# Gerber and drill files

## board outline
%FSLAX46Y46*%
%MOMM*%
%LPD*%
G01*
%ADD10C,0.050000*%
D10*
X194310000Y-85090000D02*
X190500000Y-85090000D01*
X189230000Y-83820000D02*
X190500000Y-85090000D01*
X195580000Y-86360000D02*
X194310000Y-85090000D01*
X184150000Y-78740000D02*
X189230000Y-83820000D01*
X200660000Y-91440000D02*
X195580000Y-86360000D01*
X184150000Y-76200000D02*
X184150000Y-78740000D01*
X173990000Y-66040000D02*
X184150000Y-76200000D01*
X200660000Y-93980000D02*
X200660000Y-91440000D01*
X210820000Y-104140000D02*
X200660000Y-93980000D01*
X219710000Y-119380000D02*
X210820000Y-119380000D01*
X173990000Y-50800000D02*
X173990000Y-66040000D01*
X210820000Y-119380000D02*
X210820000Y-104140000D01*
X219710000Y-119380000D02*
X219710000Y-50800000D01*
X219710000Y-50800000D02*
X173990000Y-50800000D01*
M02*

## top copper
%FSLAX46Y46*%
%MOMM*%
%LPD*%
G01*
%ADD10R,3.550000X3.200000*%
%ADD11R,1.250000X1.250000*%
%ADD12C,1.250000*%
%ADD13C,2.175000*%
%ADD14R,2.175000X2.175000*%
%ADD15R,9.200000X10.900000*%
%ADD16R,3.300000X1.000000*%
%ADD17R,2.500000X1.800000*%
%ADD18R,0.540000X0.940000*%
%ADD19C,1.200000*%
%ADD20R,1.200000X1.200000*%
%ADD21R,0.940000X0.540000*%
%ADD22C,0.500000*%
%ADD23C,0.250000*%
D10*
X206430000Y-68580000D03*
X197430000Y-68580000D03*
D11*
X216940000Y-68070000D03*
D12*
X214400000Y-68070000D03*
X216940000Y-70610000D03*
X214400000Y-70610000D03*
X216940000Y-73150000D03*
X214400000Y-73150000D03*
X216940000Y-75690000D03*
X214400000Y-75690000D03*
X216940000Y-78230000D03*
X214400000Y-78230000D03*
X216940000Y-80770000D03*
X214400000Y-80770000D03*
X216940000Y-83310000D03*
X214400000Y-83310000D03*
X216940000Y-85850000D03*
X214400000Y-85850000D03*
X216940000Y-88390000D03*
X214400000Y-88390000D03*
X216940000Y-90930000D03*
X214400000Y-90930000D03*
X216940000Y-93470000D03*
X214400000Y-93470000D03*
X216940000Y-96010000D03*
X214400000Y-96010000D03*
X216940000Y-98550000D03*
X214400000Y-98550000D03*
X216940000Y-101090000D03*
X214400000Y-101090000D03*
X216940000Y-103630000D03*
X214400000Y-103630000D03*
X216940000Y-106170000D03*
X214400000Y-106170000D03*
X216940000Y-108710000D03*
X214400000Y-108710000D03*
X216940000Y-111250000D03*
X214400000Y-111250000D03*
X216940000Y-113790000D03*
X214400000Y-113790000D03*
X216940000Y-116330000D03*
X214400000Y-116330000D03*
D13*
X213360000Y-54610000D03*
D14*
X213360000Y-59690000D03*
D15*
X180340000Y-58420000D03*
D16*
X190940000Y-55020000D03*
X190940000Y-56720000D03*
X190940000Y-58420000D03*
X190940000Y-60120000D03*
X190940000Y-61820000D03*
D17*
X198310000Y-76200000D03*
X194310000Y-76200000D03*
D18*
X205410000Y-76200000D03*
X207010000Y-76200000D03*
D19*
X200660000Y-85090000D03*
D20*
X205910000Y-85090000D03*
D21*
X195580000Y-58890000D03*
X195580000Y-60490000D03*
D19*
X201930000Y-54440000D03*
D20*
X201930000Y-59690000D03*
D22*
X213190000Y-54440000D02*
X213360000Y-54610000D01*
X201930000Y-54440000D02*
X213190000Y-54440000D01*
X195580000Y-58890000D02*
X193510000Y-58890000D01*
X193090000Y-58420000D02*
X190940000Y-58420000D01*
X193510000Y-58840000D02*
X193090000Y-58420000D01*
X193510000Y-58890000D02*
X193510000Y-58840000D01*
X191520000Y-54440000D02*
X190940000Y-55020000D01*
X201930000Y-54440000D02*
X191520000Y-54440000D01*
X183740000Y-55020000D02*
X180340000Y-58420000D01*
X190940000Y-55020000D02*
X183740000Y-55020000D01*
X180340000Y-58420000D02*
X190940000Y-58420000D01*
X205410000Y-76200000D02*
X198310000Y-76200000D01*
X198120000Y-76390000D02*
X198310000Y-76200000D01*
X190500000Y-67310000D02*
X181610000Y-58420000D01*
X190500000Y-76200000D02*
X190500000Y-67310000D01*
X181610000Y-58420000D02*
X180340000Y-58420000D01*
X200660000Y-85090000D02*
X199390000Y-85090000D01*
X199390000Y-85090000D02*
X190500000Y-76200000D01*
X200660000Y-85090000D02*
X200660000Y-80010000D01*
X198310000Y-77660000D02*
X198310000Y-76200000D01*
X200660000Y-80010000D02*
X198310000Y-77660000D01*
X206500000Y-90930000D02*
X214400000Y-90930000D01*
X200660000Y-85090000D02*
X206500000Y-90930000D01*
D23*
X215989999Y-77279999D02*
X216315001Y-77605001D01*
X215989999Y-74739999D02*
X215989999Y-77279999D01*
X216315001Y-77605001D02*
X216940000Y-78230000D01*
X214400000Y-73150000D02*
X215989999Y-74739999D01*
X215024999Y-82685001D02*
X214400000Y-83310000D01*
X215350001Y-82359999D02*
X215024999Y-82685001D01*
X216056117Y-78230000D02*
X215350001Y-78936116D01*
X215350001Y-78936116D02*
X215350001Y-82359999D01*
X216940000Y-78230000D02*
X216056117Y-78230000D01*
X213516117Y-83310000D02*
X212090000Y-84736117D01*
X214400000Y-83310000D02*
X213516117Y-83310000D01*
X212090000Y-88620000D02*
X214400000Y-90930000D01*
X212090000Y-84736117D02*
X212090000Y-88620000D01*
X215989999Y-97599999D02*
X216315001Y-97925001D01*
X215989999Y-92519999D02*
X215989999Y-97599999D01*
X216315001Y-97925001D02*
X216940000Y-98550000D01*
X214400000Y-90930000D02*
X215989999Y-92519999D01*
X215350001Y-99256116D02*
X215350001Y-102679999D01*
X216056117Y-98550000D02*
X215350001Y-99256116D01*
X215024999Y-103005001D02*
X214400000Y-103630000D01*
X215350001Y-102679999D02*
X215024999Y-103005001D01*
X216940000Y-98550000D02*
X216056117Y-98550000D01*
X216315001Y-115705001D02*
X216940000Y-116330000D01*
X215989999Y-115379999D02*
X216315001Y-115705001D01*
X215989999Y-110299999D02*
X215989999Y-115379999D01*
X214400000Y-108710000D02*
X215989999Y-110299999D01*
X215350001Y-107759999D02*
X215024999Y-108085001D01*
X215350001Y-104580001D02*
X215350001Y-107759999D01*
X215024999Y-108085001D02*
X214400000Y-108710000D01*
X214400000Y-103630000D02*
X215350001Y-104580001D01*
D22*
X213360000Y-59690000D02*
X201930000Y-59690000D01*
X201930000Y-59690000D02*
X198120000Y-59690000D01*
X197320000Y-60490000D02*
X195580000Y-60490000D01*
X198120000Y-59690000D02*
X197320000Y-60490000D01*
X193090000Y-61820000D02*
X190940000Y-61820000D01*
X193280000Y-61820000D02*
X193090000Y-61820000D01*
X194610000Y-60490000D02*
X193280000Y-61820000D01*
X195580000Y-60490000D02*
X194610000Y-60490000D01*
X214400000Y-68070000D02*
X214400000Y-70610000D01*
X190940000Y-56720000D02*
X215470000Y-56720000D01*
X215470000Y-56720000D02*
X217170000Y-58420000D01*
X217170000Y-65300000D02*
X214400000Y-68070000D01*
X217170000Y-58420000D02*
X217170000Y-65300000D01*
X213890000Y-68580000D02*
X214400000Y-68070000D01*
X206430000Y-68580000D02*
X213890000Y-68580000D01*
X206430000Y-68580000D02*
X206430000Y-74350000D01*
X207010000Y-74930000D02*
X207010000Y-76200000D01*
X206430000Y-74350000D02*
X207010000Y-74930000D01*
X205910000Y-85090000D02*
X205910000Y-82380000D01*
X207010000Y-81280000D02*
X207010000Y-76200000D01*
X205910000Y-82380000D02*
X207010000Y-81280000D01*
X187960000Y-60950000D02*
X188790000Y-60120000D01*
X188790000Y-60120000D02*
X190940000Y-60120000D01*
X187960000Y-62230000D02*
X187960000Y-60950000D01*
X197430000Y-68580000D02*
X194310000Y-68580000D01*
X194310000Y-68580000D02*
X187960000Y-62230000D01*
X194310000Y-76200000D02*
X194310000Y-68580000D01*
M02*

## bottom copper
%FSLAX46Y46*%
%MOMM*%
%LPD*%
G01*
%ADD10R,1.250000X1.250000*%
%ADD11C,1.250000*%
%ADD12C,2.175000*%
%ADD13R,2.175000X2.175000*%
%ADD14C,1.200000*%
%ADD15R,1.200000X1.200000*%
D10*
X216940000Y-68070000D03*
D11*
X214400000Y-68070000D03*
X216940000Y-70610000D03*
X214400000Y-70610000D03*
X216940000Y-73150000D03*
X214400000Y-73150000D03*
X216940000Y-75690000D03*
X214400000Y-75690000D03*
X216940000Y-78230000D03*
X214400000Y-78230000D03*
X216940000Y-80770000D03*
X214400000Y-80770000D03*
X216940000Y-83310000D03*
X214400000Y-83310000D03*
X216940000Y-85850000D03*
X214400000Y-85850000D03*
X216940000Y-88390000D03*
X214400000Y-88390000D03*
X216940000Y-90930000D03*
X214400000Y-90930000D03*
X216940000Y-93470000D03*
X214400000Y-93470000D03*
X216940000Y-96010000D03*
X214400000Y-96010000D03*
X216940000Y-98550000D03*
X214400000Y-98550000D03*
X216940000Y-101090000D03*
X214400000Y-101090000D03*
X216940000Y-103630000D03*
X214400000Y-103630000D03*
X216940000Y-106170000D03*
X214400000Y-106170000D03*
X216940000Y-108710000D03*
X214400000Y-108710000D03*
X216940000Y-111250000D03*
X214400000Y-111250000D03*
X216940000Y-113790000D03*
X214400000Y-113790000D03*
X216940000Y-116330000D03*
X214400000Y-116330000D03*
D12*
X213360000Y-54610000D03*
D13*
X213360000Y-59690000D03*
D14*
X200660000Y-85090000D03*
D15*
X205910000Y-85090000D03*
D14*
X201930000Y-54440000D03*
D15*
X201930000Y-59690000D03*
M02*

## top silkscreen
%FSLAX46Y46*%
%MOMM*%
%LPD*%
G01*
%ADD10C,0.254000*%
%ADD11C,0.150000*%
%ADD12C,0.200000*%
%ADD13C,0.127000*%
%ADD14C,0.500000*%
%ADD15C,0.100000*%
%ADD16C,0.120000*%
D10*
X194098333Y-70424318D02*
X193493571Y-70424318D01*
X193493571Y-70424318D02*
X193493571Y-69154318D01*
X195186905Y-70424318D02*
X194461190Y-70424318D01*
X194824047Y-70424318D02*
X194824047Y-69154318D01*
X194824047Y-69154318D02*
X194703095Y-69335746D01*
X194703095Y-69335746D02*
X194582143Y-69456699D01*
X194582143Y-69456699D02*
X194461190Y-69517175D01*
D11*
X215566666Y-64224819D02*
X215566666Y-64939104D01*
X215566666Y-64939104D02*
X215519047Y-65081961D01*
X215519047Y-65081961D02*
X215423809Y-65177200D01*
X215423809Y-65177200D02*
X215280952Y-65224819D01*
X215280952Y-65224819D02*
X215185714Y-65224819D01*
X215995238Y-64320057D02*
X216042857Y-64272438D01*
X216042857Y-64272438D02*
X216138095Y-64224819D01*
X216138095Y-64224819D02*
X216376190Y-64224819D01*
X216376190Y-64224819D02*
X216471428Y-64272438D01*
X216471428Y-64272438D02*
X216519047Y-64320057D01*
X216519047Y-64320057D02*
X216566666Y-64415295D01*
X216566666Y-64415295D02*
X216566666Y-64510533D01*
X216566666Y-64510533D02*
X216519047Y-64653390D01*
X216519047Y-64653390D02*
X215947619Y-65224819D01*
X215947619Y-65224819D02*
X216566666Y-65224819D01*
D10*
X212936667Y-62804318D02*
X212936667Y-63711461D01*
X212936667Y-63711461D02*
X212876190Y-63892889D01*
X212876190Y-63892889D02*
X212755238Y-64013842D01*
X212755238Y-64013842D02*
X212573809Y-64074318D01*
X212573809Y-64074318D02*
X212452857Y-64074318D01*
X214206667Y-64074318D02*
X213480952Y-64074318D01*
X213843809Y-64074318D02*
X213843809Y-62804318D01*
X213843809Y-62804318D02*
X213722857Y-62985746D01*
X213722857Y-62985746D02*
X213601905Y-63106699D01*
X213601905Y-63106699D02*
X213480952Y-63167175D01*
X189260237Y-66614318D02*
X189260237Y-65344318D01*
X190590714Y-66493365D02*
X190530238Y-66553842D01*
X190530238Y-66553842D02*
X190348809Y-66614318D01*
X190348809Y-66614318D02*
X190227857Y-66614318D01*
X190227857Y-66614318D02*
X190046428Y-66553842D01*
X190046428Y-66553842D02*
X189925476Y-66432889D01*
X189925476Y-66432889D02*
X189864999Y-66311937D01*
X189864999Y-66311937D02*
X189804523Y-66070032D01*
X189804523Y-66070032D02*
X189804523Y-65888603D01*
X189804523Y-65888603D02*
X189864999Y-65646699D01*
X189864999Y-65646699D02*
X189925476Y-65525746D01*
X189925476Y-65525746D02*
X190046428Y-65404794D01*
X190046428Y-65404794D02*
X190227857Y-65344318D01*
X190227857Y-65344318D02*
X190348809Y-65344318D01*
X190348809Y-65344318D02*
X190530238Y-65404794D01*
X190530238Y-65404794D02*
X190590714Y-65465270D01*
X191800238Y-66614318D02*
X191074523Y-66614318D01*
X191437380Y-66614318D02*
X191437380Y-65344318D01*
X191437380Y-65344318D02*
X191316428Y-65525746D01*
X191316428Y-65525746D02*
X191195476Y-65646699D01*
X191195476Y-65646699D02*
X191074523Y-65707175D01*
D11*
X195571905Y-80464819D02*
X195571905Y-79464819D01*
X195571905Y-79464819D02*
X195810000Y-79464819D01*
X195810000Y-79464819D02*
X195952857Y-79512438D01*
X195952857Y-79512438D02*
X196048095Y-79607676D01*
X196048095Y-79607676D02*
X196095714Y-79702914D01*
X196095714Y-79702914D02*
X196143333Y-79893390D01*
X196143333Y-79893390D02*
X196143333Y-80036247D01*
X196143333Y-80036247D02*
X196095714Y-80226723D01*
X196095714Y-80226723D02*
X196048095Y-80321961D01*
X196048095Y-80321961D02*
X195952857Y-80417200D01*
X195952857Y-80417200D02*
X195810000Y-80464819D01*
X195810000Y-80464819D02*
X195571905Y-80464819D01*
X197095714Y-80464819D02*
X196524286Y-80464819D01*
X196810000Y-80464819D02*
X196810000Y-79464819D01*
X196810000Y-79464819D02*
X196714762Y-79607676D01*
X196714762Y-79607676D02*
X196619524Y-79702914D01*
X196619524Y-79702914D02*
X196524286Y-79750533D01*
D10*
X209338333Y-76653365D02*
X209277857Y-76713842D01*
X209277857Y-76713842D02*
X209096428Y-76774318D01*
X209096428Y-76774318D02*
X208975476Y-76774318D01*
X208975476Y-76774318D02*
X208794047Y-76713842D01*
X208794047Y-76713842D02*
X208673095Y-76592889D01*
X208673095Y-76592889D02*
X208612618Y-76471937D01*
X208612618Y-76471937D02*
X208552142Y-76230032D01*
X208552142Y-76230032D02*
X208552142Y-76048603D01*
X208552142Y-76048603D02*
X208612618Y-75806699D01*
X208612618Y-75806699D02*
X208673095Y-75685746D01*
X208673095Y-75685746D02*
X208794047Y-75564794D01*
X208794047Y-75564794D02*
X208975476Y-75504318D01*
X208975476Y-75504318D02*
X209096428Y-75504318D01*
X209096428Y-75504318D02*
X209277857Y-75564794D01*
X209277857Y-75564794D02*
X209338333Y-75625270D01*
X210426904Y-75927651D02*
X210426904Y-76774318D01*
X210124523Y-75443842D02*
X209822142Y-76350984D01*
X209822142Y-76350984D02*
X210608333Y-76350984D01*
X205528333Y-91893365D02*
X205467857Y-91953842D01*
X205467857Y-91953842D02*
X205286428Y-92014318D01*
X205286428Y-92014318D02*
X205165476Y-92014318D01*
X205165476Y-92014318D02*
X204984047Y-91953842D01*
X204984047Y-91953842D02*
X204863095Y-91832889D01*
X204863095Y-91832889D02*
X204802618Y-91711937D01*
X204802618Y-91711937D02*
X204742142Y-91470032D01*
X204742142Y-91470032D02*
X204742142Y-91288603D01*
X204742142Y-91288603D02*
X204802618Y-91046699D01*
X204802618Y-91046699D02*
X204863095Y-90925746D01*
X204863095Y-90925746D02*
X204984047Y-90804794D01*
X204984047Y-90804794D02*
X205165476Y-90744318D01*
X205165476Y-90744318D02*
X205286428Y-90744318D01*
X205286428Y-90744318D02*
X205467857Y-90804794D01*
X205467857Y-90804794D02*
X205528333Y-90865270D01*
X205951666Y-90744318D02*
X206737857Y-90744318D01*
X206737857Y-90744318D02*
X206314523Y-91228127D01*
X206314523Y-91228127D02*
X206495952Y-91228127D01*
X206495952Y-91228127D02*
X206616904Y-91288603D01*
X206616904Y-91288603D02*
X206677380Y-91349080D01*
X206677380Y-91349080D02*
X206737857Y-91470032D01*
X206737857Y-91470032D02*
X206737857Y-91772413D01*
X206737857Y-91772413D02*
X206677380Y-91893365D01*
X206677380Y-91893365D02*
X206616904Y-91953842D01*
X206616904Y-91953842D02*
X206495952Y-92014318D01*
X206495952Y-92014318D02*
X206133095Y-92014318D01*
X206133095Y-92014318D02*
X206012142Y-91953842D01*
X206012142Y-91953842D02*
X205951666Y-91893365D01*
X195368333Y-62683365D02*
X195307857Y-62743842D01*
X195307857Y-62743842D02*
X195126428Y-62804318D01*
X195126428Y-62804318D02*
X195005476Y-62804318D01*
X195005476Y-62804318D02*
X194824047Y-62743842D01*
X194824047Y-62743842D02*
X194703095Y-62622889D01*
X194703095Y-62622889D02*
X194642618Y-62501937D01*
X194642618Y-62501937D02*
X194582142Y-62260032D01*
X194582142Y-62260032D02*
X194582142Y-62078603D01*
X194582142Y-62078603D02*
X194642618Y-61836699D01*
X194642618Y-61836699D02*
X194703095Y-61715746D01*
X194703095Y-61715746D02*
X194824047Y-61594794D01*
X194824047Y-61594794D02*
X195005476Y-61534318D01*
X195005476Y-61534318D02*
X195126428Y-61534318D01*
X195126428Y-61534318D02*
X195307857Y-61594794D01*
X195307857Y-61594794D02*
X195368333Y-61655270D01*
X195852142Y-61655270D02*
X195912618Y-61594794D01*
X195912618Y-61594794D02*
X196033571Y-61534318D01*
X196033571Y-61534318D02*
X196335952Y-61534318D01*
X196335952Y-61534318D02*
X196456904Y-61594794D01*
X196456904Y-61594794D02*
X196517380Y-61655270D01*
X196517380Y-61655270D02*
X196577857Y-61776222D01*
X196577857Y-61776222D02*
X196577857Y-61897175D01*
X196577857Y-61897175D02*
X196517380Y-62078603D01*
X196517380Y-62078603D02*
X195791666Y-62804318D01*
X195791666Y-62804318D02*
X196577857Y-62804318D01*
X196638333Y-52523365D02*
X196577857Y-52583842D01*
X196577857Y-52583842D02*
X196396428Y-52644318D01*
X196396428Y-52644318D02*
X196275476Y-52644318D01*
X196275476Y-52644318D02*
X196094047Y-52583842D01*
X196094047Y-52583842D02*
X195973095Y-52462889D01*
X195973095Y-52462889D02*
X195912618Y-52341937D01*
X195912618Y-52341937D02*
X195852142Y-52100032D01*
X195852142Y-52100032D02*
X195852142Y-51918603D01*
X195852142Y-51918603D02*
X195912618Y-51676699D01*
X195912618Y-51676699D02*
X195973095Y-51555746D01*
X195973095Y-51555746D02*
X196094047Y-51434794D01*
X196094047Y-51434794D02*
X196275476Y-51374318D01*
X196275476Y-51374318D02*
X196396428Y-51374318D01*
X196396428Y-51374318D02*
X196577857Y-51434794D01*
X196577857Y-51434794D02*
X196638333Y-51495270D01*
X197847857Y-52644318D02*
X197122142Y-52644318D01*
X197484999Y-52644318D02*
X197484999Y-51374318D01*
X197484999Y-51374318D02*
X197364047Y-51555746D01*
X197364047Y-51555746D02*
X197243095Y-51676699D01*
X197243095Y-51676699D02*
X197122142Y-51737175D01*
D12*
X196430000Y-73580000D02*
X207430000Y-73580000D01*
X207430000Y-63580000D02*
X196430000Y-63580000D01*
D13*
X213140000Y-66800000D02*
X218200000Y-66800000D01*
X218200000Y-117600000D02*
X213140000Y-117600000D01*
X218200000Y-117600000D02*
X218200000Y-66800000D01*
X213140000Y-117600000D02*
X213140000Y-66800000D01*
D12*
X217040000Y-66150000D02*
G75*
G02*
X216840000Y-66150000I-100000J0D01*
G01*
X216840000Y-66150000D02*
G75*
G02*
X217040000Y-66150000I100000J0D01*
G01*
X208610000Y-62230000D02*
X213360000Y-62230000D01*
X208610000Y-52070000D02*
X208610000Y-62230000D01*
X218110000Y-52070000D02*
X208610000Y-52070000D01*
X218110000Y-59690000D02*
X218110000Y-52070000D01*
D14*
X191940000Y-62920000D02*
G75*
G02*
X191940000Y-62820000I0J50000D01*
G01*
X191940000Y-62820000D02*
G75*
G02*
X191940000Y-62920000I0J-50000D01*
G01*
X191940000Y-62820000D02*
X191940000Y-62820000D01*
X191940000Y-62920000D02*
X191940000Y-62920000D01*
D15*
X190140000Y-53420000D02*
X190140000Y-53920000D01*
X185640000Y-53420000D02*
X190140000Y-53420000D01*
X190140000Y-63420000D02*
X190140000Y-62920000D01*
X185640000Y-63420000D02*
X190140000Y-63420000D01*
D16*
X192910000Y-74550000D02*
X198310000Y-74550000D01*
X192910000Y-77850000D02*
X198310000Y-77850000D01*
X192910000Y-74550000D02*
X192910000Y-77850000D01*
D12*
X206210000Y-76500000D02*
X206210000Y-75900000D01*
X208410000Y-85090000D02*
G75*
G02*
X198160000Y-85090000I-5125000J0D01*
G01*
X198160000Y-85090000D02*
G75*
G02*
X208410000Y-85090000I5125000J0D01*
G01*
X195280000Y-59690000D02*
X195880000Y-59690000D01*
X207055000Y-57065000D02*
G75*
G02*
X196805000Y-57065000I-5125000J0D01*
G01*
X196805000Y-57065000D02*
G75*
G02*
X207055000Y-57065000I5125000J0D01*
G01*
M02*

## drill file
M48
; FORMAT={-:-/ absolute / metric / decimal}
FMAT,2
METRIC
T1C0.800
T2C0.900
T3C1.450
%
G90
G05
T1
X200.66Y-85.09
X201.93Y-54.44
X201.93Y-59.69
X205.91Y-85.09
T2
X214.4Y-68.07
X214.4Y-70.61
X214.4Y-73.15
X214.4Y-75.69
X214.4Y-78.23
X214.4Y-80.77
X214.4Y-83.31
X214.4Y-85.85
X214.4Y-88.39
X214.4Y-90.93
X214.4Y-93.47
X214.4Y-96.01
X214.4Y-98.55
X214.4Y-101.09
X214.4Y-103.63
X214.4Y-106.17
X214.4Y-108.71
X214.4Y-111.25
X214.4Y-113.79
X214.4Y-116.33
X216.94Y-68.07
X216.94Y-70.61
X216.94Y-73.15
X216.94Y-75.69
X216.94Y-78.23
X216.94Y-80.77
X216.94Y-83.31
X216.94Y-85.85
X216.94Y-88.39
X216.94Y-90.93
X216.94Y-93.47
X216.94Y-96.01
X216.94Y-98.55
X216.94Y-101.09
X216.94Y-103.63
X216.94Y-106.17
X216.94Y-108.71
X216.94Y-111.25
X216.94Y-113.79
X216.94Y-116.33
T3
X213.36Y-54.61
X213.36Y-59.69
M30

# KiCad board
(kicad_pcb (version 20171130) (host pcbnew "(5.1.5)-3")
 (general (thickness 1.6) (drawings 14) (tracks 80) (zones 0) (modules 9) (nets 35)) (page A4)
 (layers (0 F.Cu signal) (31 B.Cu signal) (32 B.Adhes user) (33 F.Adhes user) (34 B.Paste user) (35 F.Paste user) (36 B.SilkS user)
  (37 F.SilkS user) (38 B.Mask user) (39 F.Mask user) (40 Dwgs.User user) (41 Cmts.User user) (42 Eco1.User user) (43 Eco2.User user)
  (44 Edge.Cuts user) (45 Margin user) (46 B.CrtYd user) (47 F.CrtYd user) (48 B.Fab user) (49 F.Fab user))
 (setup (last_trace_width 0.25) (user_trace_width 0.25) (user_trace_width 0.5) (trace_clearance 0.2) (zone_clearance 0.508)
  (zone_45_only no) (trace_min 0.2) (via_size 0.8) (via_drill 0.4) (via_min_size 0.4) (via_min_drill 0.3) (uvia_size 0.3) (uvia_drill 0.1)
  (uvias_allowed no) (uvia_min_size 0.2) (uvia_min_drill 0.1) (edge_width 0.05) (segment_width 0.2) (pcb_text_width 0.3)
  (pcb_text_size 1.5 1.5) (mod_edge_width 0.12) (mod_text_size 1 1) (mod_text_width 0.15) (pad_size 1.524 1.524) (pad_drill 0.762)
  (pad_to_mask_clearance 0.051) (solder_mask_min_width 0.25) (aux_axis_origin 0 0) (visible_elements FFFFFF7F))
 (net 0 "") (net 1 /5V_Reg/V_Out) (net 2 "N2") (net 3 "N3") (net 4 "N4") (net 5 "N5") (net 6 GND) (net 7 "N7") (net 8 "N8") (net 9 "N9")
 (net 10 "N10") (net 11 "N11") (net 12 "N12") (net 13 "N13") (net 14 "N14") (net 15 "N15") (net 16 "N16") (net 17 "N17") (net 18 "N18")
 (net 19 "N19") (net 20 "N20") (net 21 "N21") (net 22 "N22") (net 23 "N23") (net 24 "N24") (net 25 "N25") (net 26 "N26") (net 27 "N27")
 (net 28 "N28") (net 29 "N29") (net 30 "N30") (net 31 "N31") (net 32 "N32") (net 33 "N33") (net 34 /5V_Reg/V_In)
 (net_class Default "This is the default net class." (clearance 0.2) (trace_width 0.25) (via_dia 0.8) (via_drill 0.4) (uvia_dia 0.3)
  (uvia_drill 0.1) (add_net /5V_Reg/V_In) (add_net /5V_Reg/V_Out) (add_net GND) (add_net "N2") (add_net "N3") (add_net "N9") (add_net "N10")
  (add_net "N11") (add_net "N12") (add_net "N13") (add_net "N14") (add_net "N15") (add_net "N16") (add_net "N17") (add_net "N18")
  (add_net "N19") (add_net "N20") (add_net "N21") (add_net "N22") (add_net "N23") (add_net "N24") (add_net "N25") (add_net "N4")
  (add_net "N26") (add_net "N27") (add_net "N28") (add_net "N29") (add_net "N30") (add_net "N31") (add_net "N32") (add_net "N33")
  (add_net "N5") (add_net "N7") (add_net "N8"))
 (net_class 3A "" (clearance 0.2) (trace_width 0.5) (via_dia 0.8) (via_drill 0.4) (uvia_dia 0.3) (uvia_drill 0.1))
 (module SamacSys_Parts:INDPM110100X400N (layer F.Cu) (at 201.93 68.58)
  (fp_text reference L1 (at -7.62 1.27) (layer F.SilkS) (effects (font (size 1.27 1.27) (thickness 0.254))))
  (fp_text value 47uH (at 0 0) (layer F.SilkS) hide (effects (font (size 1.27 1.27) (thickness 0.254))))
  (fp_line (start -5.5 5) (end 5.5 5) (layer F.SilkS) (width 0.2))
  (fp_line (start 5.5 -5) (end -5.5 -5) (layer F.SilkS) (width 0.2))
  (pad 2 smd rect (at 4.5 0 90) (size 3.2 3.55) (layers F.Cu F.Paste F.Mask) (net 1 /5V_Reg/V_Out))
  (pad 1 smd rect (at -4.5 0 90) (size 3.2 3.55) (layers F.Cu F.Paste F.Mask) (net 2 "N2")))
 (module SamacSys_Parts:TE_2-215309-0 (layer F.Cu) (at 216.94 68.07 270)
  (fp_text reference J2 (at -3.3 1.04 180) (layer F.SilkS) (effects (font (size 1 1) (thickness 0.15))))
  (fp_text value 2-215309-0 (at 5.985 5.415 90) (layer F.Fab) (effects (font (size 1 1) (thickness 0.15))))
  (fp_line (start -1.27 3.8) (end -1.27 -1.26) (layer F.SilkS) (width 0.127))
  (fp_line (start 49.53 -1.26) (end 49.53 3.8) (layer F.SilkS) (width 0.127))
  (fp_line (start 49.53 -1.26) (end -1.27 -1.26) (layer F.SilkS) (width 0.127))
  (fp_line (start 49.53 3.8) (end -1.27 3.8) (layer F.SilkS) (width 0.127))
  (fp_circle (center -1.92 0) (end -1.82 0) (layer F.SilkS) (width 0.2))
  (pad 1 thru_hole rect (at 0 0 270) (size 1.25 1.25) (drill 0.9) (layers *.Cu *.Mask) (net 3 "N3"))
  (pad 2 thru_hole circle (at 0 2.54 270) (size 1.25 1.25) (drill 0.9) (layers *.Cu *.Mask) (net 1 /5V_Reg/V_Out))
  (pad 3 thru_hole circle (at 2.54 0 270) (size 1.25 1.25) (drill 0.9) (layers *.Cu *.Mask) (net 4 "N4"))
  (pad 4 thru_hole circle (at 2.54 2.54 270) (size 1.25 1.25) (drill 0.9) (layers *.Cu *.Mask) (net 1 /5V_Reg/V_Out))
  (pad 5 thru_hole circle (at 5.08 0 270) (size 1.25 1.25) (drill 0.9) (layers *.Cu *.Mask) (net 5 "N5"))
  (pad 6 thru_hole circle (at 5.08 2.54 270) (size 1.25 1.25) (drill 0.9) (layers *.Cu *.Mask) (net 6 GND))
  (pad 7 thru_hole circle (at 7.62 0 270) (size 1.25 1.25) (drill 0.9) (layers *.Cu *.Mask) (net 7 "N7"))
  (pad 8 thru_hole circle (at 7.62 2.54 270) (size 1.25 1.25) (drill 0.9) (layers *.Cu *.Mask) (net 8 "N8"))
  (pad 9 thru_hole circle (at 10.16 0 270) (size 1.25 1.25) (drill 0.9) (layers *.Cu *.Mask) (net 6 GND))
  (pad 10 thru_hole circle (at 10.16 2.54 270) (size 1.25 1.25) (drill 0.9) (layers *.Cu *.Mask) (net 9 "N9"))
  (pad 11 thru_hole circle (at 12.7 0 270) (size 1.25 1.25) (drill 0.9) (layers *.Cu *.Mask) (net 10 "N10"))
  (pad 12 thru_hole circle (at 12.7 2.54 270) (size 1.25 1.25) (drill 0.9) (layers *.Cu *.Mask) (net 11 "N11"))
  (pad 13 thru_hole circle (at 15.24 0 270) (size 1.25 1.25) (drill 0.9) (layers *.Cu *.Mask) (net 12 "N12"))
  (pad 14 thru_hole circle (at 15.24 2.54 270) (size 1.25 1.25) (drill 0.9) (layers *.Cu *.Mask) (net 6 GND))
  (pad 15 thru_hole circle (at 17.78 0 270) (size 1.25 1.25) (drill 0.9) (layers *.Cu *.Mask) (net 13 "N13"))
  (pad 16 thru_hole circle (at 17.78 2.54 270) (size 1.25 1.25) (drill 0.9) (layers *.Cu *.Mask) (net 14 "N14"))
  (pad 17 thru_hole circle (at 20.32 0 270) (size 1.25 1.25) (drill 0.9) (layers *.Cu *.Mask) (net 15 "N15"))
  (pad 18 thru_hole circle (at 20.32 2.54 270) (size 1.25 1.25) (drill 0.9) (layers *.Cu *.Mask) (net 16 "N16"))
  (pad 19 thru_hole circle (at 22.86 0 270) (size 1.25 1.25) (drill 0.9) (layers *.Cu *.Mask) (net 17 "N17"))
  (pad 20 thru_hole circle (at 22.86 2.54 270) (size 1.25 1.25) (drill 0.9) (layers *.Cu *.Mask) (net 6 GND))
  (pad 21 thru_hole circle (at 25.4 0 270) (size 1.25 1.25) (drill 0.9) (layers *.Cu *.Mask) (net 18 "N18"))
  (pad 22 thru_hole circle (at 25.4 2.54 270) (size 1.25 1.25) (drill 0.9) (layers *.Cu *.Mask) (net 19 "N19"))
  (pad 23 thru_hole circle (at 27.94 0 270) (size 1.25 1.25) (drill 0.9) (layers *.Cu *.Mask) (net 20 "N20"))
  (pad 24 thru_hole circle (at 27.94 2.54 270) (size 1.25 1.25) (drill 0.9) (layers *.Cu *.Mask) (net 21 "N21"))
  (pad 25 thru_hole circle (at 30.48 0 270) (size 1.25 1.25) (drill 0.9) (layers *.Cu *.Mask) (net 6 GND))
  (pad 26 thru_hole circle (at 30.48 2.54 270) (size 1.25 1.25) (drill 0.9) (layers *.Cu *.Mask) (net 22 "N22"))
  (pad 27 thru_hole circle (at 33.02 0 270) (size 1.25 1.25) (drill 0.9) (layers *.Cu *.Mask) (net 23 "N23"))
  (pad 28 thru_hole circle (at 33.02 2.54 270) (size 1.25 1.25) (drill 0.9) (layers *.Cu *.Mask) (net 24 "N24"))
  (pad 29 thru_hole circle (at 35.56 0 270) (size 1.25 1.25) (drill 0.9) (layers *.Cu *.Mask) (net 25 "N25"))
  (pad 30 thru_hole circle (at 35.56 2.54 270) (size 1.25 1.25) (drill 0.9) (layers *.Cu *.Mask) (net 6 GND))
  (pad 31 thru_hole circle (at 38.1 0 270) (size 1.25 1.25) (drill 0.9) (layers *.Cu *.Mask) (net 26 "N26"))
  (pad 32 thru_hole circle (at 38.1 2.54 270) (size 1.25 1.25) (drill 0.9) (layers *.Cu *.Mask) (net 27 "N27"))
  (pad 33 thru_hole circle (at 40.64 0 270) (size 1.25 1.25) (drill 0.9) (layers *.Cu *.Mask) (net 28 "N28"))
  (pad 34 thru_hole circle (at 40.64 2.54 270) (size 1.25 1.25) (drill 0.9) (layers *.Cu *.Mask) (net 6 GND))
  (pad 35 thru_hole circle (at 43.18 0 270) (size 1.25 1.25) (drill 0.9) (layers *.Cu *.Mask) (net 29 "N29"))
  (pad 36 thru_hole circle (at 43.18 2.54 270) (size 1.25 1.25) (drill 0.9) (layers *.Cu *.Mask) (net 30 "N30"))
  (pad 37 thru_hole circle (at 45.72 0 270) (size 1.25 1.25) (drill 0.9) (layers *.Cu *.Mask) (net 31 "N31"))
  (pad 38 thru_hole circle (at 45.72 2.54 270) (size 1.25 1.25) (drill 0.9) (layers *.Cu *.Mask) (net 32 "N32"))
  (pad 39 thru_hole circle (at 48.26 0 270) (size 1.25 1.25) (drill 0.9) (layers *.Cu *.Mask) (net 6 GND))
  (pad 40 thru_hole circle (at 48.26 2.54 270) (size 1.25 1.25) (drill 0.9) (layers *.Cu *.Mask) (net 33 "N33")))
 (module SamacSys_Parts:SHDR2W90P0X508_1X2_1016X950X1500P (layer F.Cu) (at 213.36 59.69 90)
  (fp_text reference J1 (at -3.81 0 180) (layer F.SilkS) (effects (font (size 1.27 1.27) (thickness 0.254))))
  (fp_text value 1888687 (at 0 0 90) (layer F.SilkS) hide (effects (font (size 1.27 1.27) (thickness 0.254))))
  (fp_line (start -2.54 -4.75) (end -2.54 0) (layer F.SilkS) (width 0.2))
  (fp_line (start 7.62 -4.75) (end -2.54 -4.75) (layer F.SilkS) (width 0.2))
  (fp_line (start 7.62 4.75) (end 7.62 -4.75) (layer F.SilkS) (width 0.2))
  (fp_line (start 0 4.75) (end 7.62 4.75) (layer F.SilkS) (width 0.2))
  (pad 2 thru_hole circle (at 5.08 0 90) (size 2.175 2.175) (drill 1.45) (layers *.Cu *.Mask) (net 6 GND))
  (pad 1 thru_hole rect (at 0 0 90) (size 2.175 2.175) (drill 1.45) (layers *.Cu *.Mask) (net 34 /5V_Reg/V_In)))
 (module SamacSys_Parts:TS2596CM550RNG (layer F.Cu) (at 185.64 58.42 90)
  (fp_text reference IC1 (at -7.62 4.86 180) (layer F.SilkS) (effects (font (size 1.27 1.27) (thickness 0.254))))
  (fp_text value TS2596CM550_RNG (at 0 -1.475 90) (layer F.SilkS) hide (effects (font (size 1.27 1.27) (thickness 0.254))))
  (fp_arc (start -4.45 6.3) (end -4.4 6.3) (angle -180) (layer F.SilkS) (width 0.5))
  (fp_arc (start -4.45 6.3) (end -4.5 6.3) (angle -180) (layer F.SilkS) (width 0.5))
  (fp_line (start -4.4 6.3) (end -4.4 6.3) (layer F.SilkS) (width 0.5))
  (fp_line (start -4.5 6.3) (end -4.5 6.3) (layer F.SilkS) (width 0.5))
  (fp_line (start 5 4.5) (end 4.5 4.5) (layer F.SilkS) (width 0.1))
  (fp_line (start 5 0) (end 5 4.5) (layer F.SilkS) (width 0.1))
  (fp_line (start -5 4.5) (end -4.5 4.5) (layer F.SilkS) (width 0.1))
  (fp_line (start -5 0) (end -5 4.5) (layer F.SilkS) (width 0.1))
  (pad 6 smd rect (at 0 -5.3 180) (size 9.2 10.9) (layers F.Cu F.Paste F.Mask) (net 6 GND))
  (pad 5 smd rect (at 3.4 5.3 90) (size 1 3.3) (layers F.Cu F.Paste F.Mask) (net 6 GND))
  (pad 4 smd rect (at 1.7 5.3 90) (size 1 3.3) (layers F.Cu F.Paste F.Mask) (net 1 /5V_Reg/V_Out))
  (pad 3 smd rect (at 0 5.3 90) (size 1 3.3) (layers F.Cu F.Paste F.Mask) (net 6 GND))
  (pad 2 smd rect (at -1.7 5.3 90) (size 1 3.3) (layers F.Cu F.Paste F.Mask) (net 2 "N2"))
  (pad 1 smd rect (at -3.4 5.3 90) (size 1 3.3) (layers F.Cu F.Paste F.Mask) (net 34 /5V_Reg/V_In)))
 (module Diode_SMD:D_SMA (layer F.Cu) (at 196.31 76.2)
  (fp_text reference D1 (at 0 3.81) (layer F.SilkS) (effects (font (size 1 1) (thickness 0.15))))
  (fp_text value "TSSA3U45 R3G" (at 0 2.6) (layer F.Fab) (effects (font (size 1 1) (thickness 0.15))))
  (fp_line (start -3.4 -1.65) (end 2 -1.65) (layer F.SilkS) (width 0.12))
  (fp_line (start -3.4 1.65) (end 2 1.65) (layer F.SilkS) (width 0.12))
  (fp_line (start -3.4 -1.65) (end -3.4 1.65) (layer F.SilkS) (width 0.12))
  (pad 2 smd rect (at 2 0) (size 2.5 1.8) (layers F.Cu F.Paste F.Mask) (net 6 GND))
  (pad 1 smd rect (at -2 0) (size 2.5 1.8) (layers F.Cu F.Paste F.Mask) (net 2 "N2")))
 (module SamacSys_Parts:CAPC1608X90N (layer F.Cu) (at 206.21 76.2 180)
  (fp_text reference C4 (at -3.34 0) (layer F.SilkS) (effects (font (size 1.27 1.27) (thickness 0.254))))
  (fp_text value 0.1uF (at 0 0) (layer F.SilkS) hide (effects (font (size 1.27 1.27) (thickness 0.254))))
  (fp_line (start 0 -0.3) (end 0 0.3) (layer F.SilkS) (width 0.2))
  (pad 2 smd rect (at 0.8 0 180) (size 0.54 0.94) (layers F.Cu F.Paste F.Mask) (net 6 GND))
  (pad 1 smd rect (at -0.8 0 180) (size 0.54 0.94) (layers F.Cu F.Paste F.Mask) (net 1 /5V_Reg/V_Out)))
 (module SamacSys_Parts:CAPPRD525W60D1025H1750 (layer F.Cu) (at 205.91 85.09 180)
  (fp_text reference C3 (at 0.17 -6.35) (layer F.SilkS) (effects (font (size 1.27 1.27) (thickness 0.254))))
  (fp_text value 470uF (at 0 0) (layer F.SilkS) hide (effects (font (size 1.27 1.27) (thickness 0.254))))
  (fp_circle (center 2.625 0) (end 2.625 5.125) (layer F.SilkS) (width 0.2))
  (pad 2 thru_hole circle (at 5.25 0 180) (size 1.2 1.2) (drill 0.8) (layers *.Cu *.Mask) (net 6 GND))
  (pad 1 thru_hole rect (at 0 0 180) (size 1.2 1.2) (drill 0.8) (layers *.Cu *.Mask) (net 1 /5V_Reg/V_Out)))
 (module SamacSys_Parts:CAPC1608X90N (layer F.Cu) (at 195.58 59.69 90)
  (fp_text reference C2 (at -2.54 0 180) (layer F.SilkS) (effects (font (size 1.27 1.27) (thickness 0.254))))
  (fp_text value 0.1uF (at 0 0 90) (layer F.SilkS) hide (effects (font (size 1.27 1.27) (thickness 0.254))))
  (fp_line (start 0 -0.3) (end 0 0.3) (layer F.SilkS) (width 0.2))
  (pad 2 smd rect (at 0.8 0 90) (size 0.54 0.94) (layers F.Cu F.Paste F.Mask) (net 6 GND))
  (pad 1 smd rect (at -0.8 0 90) (size 0.54 0.94) (layers F.Cu F.Paste F.Mask) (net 34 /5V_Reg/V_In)))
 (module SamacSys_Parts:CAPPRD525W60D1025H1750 (layer F.Cu) (at 201.93 59.69 90)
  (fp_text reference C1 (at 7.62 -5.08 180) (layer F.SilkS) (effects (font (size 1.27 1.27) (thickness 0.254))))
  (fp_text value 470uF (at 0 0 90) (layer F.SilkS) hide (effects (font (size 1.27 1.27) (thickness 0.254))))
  (fp_circle (center 2.625 0) (end 2.625 5.125) (layer F.SilkS) (width 0.2))
  (pad 2 thru_hole circle (at 5.25 0 90) (size 1.2 1.2) (drill 0.8) (layers *.Cu *.Mask) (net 6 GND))
  (pad 1 thru_hole rect (at 0 0 90) (size 1.2 1.2) (drill 0.8) (layers *.Cu *.Mask) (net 34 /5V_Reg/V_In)))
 (gr_line (start 194.31 85.09) (end 190.5 85.09) (layer Edge.Cuts) (width 0.05))
 (gr_line (start 189.23 83.82) (end 190.5 85.09) (layer Edge.Cuts) (width 0.05))
 (gr_line (start 195.58 86.36) (end 194.31 85.09) (layer Edge.Cuts) (width 0.05))
 (gr_line (start 184.15 78.74) (end 189.23 83.82) (layer Edge.Cuts) (width 0.05))
 (gr_line (start 200.66 91.44) (end 195.58 86.36) (layer Edge.Cuts) (width 0.05))
 (gr_line (start 184.15 76.2) (end 184.15 78.74) (layer Edge.Cuts) (width 0.05))
 (gr_line (start 173.99 66.04) (end 184.15 76.2) (layer Edge.Cuts) (width 0.05))
 (gr_line (start 200.66 93.98) (end 200.66 91.44) (layer Edge.Cuts) (width 0.05))
 (gr_line (start 210.82 104.14) (end 200.66 93.98) (layer Edge.Cuts) (width 0.05))
 (gr_line (start 219.71 119.38) (end 210.82 119.38) (layer Edge.Cuts) (width 0.05))
 (gr_line (start 173.99 50.8) (end 173.99 66.04) (layer Edge.Cuts) (width 0.05))
 (gr_line (start 210.82 119.38) (end 210.82 104.14) (layer Edge.Cuts) (width 0.05))
 (gr_line (start 219.71 119.38) (end 219.71 50.8) (layer Edge.Cuts) (width 0.05))
 (gr_line (start 219.71 50.8) (end 173.99 50.8) (layer Edge.Cuts) (width 0.05))
 (segment (start 213.19 54.44) (end 213.36 54.61) (width 0.5) (layer F.Cu) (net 6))
 (segment (start 201.93 54.44) (end 213.19 54.44) (width 0.5) (layer F.Cu) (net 6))
 (segment (start 195.58 58.89) (end 193.51 58.89) (width 0.5) (layer F.Cu) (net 6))
 (segment (start 193.09 58.42) (end 190.94 58.42) (width 0.5) (layer F.Cu) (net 6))
 (segment (start 193.51 58.84) (end 193.09 58.42) (width 0.5) (layer F.Cu) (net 6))
 (segment (start 193.51 58.89) (end 193.51 58.84) (width 0.5) (layer F.Cu) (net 6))
 (segment (start 191.52 54.44) (end 190.94 55.02) (width 0.5) (layer F.Cu) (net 6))
 (segment (start 201.93 54.44) (end 191.52 54.44) (width 0.5) (layer F.Cu) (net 6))
 (segment (start 183.74 55.02) (end 180.34 58.42) (width 0.5) (layer F.Cu) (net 6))
 (segment (start 190.94 55.02) (end 183.74 55.02) (width 0.5) (layer F.Cu) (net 6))
 (segment (start 180.34 58.42) (end 190.94 58.42) (width 0.5) (layer F.Cu) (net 6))
 (segment (start 205.41 76.2) (end 198.31 76.2) (width 0.5) (layer F.Cu) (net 6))
 (segment (start 198.12 76.39) (end 198.31 76.2) (width 0.5) (layer F.Cu) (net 6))
 (segment (start 190.5 67.31) (end 181.61 58.42) (width 0.5) (layer F.Cu) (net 6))
 (segment (start 190.5 76.2) (end 190.5 67.31) (width 0.5) (layer F.Cu) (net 6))
 (segment (start 181.61 58.42) (end 180.34 58.42) (width 0.5) (layer F.Cu) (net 6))
 (segment (start 200.66 85.09) (end 199.39 85.09) (width 0.5) (layer F.Cu) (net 6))
 (segment (start 199.39 85.09) (end 190.5 76.2) (width 0.5) (layer F.Cu) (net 6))
 (segment (start 200.66 85.09) (end 200.66 80.01) (width 0.5) (layer F.Cu) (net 6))
 (segment (start 198.31 77.66) (end 198.31 76.2) (width 0.5) (layer F.Cu) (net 6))
 (segment (start 200.66 80.01) (end 198.31 77.66) (width 0.5) (layer F.Cu) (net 6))
 (segment (start 206.5 90.93) (end 214.4 90.93) (width 0.5) (layer F.Cu) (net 6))
 (segment (start 200.66 85.09) (end 206.5 90.93) (width 0.5) (layer F.Cu) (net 6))
 (segment (start 215.989999 77.279999) (end 216.315001 77.605001) (width 0.25) (layer F.Cu) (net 6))
 (segment (start 215.989999 74.739999) (end 215.989999 77.279999) (width 0.25) (layer F.Cu) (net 6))
 (segment (start 216.315001 77.605001) (end 216.94 78.23) (width 0.25) (layer F.Cu) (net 6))
 (segment (start 214.4 73.15) (end 215.989999 74.739999) (width 0.25) (layer F.Cu) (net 6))
 (segment (start 215.024999 82.685001) (end 214.4 83.31) (width 0.25) (layer F.Cu) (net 6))
 (segment (start 215.350001 82.359999) (end 215.024999 82.685001) (width 0.25) (layer F.Cu) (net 6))
 (segment (start 216.056117 78.23) (end 215.350001 78.936116) (width 0.25) (layer F.Cu) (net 6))
 (segment (start 215.350001 78.936116) (end 215.350001 82.359999) (width 0.25) (layer F.Cu) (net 6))
 (segment (start 216.94 78.23) (end 216.056117 78.23) (width 0.25) (layer F.Cu) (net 6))
 (segment (start 213.516117 83.31) (end 212.09 84.736117) (width 0.25) (layer F.Cu) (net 6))
 (segment (start 214.4 83.31) (end 213.516117 83.31) (width 0.25) (layer F.Cu) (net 6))
 (segment (start 212.09 88.62) (end 214.4 90.93) (width 0.25) (layer F.Cu) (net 6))
 (segment (start 212.09 84.736117) (end 212.09 88.62) (width 0.25) (layer F.Cu) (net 6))
 (segment (start 215.989999 97.599999) (end 216.315001 97.925001) (width 0.25) (layer F.Cu) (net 6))
 (segment (start 215.989999 92.519999) (end 215.989999 97.599999) (width 0.25) (layer F.Cu) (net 6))
 (segment (start 216.315001 97.925001) (end 216.94 98.55) (width 0.25) (layer F.Cu) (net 6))
 (segment (start 214.4 90.93) (end 215.989999 92.519999) (width 0.25) (layer F.Cu) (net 6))
 (segment (start 215.350001 99.256116) (end 215.350001 102.679999) (width 0.25) (layer F.Cu) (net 6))
 (segment (start 216.056117 98.55) (end 215.350001 99.256116) (width 0.25) (layer F.Cu) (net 6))
 (segment (start 215.024999 103.005001) (end 214.4 103.63) (width 0.25) (layer F.Cu) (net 6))
 (segment (start 215.350001 102.679999) (end 215.024999 103.005001) (width 0.25) (layer F.Cu) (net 6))
 (segment (start 216.94 98.55) (end 216.056117 98.55) (width 0.25) (layer F.Cu) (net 6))
 (segment (start 216.315001 115.705001) (end 216.94 116.33) (width 0.25) (layer F.Cu) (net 6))
 (segment (start 215.989999 115.379999) (end 216.315001 115.705001) (width 0.25) (layer F.Cu) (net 6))
 (segment (start 215.989999 110.299999) (end 215.989999 115.379999) (width 0.25) (layer F.Cu) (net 6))
 (segment (start 214.4 108.71) (end 215.989999 110.299999) (width 0.25) (layer F.Cu) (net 6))
 (segment (start 215.350001 107.759999) (end 215.024999 108.085001) (width 0.25) (layer F.Cu) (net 6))
 (segment (start 215.350001 104.580001) (end 215.350001 107.759999) (width 0.25) (layer F.Cu) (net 6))
 (segment (start 215.024999 108.085001) (end 214.4 108.71) (width 0.25) (layer F.Cu) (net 6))
 (segment (start 214.4 103.63) (end 215.350001 104.580001) (width 0.25) (layer F.Cu) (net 6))
 (segment (start 213.36 59.69) (end 201.93 59.69) (width 0.5) (layer F.Cu) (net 34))
 (segment (start 201.93 59.69) (end 198.12 59.69) (width 0.5) (layer F.Cu) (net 34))
 (segment (start 197.32 60.49) (end 195.58 60.49) (width 0.5) (layer F.Cu) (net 34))
 (segment (start 198.12 59.69) (end 197.32 60.49) (width 0.5) (layer F.Cu) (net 34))
 (segment (start 193.09 61.82) (end 190.94 61.82) (width 0.5) (layer F.Cu) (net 34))
 (segment (start 193.28 61.82) (end 193.09 61.82) (width 0.5) (layer F.Cu) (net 34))
 (segment (start 194.61 60.49) (end 193.28 61.82) (width 0.5) (layer F.Cu) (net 34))
 (segment (start 195.58 60.49) (end 194.61 60.49) (width 0.5) (layer F.Cu) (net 34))
 (segment (start 214.4 68.07) (end 214.4 70.61) (width 0.5) (layer F.Cu) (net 1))
 (segment (start 190.94 56.72) (end 215.47 56.72) (width 0.5) (layer F.Cu) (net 1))
 (segment (start 215.47 56.72) (end 217.17 58.42) (width 0.5) (layer F.Cu) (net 1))
 (segment (start 217.17 65.3) (end 214.4 68.07) (width 0.5) (layer F.Cu) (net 1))
 (segment (start 217.17 58.42) (end 217.17 65.3) (width 0.5) (layer F.Cu) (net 1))
 (segment (start 213.89 68.58) (end 214.4 68.07) (width 0.5) (layer F.Cu) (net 1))
 (segment (start 206.43 68.58) (end 213.89 68.58) (width 0.5) (layer F.Cu) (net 1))
 (segment (start 206.43 68.58) (end 206.43 74.35) (width 0.5) (layer F.Cu) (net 1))
 (segment (start 207.01 74.93) (end 207.01 76.2) (width 0.5) (layer F.Cu) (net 1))
 (segment (start 206.43 74.35) (end 207.01 74.93) (width 0.5) (layer F.Cu) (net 1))
 (segment (start 205.91 85.09) (end 205.91 82.38) (width 0.5) (layer F.Cu) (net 1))
 (segment (start 207.01 81.28) (end 207.01 76.2) (width 0.5) (layer F.Cu) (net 1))
 (segment (start 205.91 82.38) (end 207.01 81.28) (width 0.5) (layer F.Cu) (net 1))
 (segment (start 187.96 60.95) (end 188.79 60.12) (width 0.5) (layer F.Cu) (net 2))
 (segment (start 188.79 60.12) (end 190.94 60.12) (width 0.5) (layer F.Cu) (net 2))
 (segment (start 187.96 62.23) (end 187.96 60.95) (width 0.5) (layer F.Cu) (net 2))
 (segment (start 197.43 68.58) (end 194.31 68.58) (width 0.5) (layer F.Cu) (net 2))
 (segment (start 194.31 68.58) (end 187.96 62.23) (width 0.5) (layer F.Cu) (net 2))
 (segment (start 194.31 76.2) (end 194.31 68.58) (width 0.5) (layer F.Cu) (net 2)))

